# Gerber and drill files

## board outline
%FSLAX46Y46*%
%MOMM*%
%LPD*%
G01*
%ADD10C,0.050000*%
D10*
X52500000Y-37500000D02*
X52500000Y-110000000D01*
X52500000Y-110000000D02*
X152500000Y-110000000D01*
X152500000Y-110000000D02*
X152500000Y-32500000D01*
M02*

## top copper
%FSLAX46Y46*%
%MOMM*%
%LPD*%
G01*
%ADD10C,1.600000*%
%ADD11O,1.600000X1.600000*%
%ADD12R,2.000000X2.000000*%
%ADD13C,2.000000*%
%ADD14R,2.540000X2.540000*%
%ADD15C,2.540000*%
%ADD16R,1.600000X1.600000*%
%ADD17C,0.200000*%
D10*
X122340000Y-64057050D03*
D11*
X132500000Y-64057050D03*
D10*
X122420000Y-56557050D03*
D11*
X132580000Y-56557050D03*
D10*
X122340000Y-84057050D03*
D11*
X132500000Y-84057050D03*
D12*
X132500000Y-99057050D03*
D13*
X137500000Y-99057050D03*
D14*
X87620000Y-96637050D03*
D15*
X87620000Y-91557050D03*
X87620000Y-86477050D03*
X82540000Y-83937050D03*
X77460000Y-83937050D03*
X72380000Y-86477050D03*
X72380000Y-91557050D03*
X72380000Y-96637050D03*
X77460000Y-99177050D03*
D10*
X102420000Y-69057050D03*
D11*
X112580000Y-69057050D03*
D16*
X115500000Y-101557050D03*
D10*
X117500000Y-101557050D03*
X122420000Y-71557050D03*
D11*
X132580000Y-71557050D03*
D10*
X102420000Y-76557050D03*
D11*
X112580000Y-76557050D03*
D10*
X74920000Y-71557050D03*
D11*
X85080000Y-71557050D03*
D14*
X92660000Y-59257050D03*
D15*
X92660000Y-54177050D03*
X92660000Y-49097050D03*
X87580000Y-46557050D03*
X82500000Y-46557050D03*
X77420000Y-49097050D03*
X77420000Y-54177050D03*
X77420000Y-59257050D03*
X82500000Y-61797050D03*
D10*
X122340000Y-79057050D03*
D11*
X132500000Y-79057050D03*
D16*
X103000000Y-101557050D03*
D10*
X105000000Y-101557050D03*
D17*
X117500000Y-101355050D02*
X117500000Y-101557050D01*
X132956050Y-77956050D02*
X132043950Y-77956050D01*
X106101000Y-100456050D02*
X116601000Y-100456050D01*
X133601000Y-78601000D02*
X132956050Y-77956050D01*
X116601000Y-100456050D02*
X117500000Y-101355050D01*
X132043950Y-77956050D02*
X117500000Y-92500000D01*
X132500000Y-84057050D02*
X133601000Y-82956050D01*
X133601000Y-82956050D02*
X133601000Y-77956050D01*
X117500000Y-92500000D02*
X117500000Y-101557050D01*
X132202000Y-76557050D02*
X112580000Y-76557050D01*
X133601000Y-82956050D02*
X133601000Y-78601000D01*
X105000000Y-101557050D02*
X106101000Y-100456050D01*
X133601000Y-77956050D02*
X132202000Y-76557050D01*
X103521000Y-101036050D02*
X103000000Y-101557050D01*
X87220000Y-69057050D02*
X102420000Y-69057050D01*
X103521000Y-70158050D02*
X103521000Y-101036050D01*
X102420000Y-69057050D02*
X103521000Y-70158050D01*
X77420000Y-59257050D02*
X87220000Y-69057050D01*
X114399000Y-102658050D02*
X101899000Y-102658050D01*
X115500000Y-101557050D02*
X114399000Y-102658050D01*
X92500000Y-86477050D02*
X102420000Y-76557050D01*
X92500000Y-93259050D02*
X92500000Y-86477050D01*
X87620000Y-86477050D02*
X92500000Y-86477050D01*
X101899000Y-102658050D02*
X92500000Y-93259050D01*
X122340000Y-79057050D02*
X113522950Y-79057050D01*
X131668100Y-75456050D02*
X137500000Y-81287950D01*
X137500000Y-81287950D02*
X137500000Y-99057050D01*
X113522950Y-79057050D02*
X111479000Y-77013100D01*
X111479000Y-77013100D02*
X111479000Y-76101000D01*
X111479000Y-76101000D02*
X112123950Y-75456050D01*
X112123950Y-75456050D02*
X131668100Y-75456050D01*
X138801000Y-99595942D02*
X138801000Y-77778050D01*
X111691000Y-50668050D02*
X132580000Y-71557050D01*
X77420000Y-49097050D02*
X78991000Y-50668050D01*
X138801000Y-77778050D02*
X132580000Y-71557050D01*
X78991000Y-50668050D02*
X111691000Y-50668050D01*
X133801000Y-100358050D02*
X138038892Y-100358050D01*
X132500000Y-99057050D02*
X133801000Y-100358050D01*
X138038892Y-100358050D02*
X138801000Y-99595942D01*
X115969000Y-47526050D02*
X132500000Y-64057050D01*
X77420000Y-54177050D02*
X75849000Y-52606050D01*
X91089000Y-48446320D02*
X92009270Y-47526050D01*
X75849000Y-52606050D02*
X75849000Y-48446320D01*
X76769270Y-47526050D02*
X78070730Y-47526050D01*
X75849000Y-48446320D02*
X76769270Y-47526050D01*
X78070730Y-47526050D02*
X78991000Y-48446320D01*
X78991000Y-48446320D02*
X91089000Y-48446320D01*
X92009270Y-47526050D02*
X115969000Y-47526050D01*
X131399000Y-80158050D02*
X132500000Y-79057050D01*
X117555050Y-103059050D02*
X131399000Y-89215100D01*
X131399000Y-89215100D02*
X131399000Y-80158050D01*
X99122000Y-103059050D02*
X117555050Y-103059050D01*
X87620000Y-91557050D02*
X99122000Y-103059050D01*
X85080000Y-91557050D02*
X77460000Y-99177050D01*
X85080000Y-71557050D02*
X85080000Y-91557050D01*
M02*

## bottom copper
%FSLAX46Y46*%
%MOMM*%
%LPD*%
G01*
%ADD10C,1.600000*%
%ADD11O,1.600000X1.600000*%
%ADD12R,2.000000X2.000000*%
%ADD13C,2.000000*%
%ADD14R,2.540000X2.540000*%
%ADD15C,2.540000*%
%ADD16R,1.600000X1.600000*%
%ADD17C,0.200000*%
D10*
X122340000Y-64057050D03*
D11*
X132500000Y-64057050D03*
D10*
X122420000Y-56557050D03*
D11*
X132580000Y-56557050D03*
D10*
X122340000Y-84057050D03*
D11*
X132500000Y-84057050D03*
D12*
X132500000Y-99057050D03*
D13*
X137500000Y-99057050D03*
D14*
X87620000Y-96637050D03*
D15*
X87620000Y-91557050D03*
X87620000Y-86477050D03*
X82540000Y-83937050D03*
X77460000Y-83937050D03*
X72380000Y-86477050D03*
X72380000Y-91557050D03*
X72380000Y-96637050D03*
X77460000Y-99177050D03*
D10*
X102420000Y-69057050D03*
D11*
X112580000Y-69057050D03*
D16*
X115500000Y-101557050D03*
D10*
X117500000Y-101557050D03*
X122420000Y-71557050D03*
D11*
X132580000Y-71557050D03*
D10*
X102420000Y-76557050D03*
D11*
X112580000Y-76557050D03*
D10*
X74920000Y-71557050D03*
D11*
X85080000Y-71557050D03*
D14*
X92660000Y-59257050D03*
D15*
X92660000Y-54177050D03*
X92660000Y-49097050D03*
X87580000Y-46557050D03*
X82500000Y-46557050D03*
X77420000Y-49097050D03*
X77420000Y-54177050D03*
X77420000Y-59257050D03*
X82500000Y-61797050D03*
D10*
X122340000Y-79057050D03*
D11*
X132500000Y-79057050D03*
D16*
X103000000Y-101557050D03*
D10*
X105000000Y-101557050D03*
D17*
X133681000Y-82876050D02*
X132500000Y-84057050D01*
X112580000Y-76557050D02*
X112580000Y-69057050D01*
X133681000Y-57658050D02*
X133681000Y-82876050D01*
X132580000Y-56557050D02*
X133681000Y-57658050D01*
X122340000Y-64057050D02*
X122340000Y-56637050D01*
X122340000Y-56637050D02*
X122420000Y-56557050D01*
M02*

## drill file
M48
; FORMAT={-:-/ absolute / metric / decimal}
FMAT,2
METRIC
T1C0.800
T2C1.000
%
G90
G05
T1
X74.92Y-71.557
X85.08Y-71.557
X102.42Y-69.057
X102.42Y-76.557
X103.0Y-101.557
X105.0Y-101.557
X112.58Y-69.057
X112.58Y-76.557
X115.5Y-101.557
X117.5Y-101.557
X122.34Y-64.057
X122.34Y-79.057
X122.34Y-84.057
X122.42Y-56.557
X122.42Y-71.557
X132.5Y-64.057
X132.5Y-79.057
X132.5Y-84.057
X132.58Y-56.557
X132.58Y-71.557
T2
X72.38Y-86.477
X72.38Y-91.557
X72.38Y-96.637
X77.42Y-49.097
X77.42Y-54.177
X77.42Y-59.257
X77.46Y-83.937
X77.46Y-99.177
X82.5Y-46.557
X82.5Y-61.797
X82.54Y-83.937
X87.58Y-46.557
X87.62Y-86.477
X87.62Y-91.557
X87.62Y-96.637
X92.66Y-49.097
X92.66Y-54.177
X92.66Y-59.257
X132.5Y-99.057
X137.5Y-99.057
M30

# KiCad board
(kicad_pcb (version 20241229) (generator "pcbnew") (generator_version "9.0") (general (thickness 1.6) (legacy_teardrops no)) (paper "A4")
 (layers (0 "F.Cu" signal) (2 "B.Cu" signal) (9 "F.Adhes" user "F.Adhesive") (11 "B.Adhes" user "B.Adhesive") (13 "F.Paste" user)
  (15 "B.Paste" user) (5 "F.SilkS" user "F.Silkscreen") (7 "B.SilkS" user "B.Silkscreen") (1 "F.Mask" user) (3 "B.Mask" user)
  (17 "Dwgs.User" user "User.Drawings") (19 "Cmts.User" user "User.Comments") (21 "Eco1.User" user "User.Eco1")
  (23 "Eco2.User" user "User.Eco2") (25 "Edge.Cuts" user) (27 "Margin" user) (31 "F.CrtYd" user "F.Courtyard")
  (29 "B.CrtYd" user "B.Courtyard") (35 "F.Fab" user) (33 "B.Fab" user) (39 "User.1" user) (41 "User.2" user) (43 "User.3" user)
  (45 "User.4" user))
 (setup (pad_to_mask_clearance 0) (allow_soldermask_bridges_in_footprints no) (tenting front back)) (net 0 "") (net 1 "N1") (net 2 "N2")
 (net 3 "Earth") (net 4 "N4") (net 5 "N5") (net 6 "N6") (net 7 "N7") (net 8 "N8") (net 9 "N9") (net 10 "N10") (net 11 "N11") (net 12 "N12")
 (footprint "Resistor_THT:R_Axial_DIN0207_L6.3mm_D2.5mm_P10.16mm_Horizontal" (layer "F.Cu") (at 122.34 64.05705)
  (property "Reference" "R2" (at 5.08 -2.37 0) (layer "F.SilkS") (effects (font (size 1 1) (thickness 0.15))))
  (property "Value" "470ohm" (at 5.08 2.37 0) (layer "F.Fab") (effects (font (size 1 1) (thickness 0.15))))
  (pad "1" thru_hole circle (at 0 0) (size 1.6 1.6) (drill 0.8) (layers "*.Cu" "*.Mask") (remove_unused_layers no) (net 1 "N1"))
  (pad "2" thru_hole oval (at 10.16 0) (size 1.6 1.6) (drill 0.8) (layers "*.Cu" "*.Mask") (remove_unused_layers no) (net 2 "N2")))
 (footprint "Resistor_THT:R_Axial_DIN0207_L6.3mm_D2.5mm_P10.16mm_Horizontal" (layer "F.Cu") (at 122.42 56.55705)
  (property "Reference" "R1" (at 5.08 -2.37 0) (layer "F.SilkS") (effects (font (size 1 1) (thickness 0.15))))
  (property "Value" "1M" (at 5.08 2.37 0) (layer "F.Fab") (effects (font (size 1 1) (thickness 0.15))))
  (pad "1" thru_hole circle (at 0 0) (size 1.6 1.6) (drill 0.8) (layers "*.Cu" "*.Mask") (remove_unused_layers no) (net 1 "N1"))
  (pad "2" thru_hole oval (at 10.16 0) (size 1.6 1.6) (drill 0.8) (layers "*.Cu" "*.Mask") (remove_unused_layers no) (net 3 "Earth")))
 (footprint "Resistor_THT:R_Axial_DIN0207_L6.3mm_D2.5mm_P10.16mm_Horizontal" (layer "F.Cu") (at 122.34 84.05705)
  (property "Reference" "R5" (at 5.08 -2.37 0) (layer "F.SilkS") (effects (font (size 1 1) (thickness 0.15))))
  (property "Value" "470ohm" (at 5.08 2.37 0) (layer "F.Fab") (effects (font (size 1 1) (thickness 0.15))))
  (pad "1" thru_hole circle (at 0 0) (size 1.6 1.6) (drill 0.8) (layers "*.Cu" "*.Mask") (remove_unused_layers no) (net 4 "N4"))
  (pad "2" thru_hole oval (at 10.16 0) (size 1.6 1.6) (drill 0.8) (layers "*.Cu" "*.Mask") (remove_unused_layers no) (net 3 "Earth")))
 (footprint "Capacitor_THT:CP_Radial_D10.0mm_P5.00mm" (layer "F.Cu") (at 132.5 99.05705)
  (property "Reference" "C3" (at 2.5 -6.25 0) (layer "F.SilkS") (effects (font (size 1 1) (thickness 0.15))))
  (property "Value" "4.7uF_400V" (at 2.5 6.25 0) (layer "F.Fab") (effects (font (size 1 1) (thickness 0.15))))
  (pad "1" thru_hole rect (at 0 0) (size 2 2) (drill 1) (layers "*.Cu" "*.Mask") (remove_unused_layers no) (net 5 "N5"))
  (pad "2" thru_hole circle (at 5 0) (size 2 2) (drill 1) (layers "*.Cu" "*.Mask") (remove_unused_layers no) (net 4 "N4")))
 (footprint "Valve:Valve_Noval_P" (layer "F.Cu") (at 87.62 96.63705)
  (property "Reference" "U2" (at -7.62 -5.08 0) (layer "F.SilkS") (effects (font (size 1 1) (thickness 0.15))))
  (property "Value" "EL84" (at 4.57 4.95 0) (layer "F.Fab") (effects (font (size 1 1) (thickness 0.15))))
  (pad "1" thru_hole rect (at 0 0) (size 2.54 2.54) (drill 1) (layers "*.Cu" "*.Mask") (remove_unused_layers no))
  (pad "2" thru_hole circle (at 0 -5.08) (size 2.54 2.54) (drill 1) (layers "*.Cu" "*.Mask") (remove_unused_layers no) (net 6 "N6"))
  (pad "3" thru_hole circle (at 0 -10.16) (size 2.54 2.54) (drill 1) (layers "*.Cu" "*.Mask") (remove_unused_layers no) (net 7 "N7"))
  (pad "4" thru_hole circle (at -5.08 -12.7) (size 2.54 2.54) (drill 1) (layers "*.Cu" "*.Mask") (remove_unused_layers no))
  (pad "5" thru_hole circle (at -10.16 -12.7) (size 2.54 2.54) (drill 1) (layers "*.Cu" "*.Mask") (remove_unused_layers no))
  (pad "6" thru_hole circle (at -15.24 -10.16) (size 2.54 2.54) (drill 1) (layers "*.Cu" "*.Mask") (remove_unused_layers no))
  (pad "7" thru_hole circle (at -15.24 -5.08) (size 2.54 2.54) (drill 1) (layers "*.Cu" "*.Mask") (remove_unused_layers no) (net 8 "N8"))
  (pad "8" thru_hole circle (at -15.24 0) (size 2.54 2.54) (drill 1) (layers "*.Cu" "*.Mask") (remove_unused_layers no))
  (pad "9" thru_hole circle (at -10.16 2.54) (size 2.54 2.54) (drill 1) (layers "*.Cu" "*.Mask") (remove_unused_layers no) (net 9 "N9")))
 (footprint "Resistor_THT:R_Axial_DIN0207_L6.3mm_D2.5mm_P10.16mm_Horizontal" (layer "F.Cu") (at 102.42 69.05705)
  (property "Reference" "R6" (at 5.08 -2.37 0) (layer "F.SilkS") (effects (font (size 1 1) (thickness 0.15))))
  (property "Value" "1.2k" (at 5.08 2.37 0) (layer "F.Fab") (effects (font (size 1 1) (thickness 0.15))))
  (pad "1" thru_hole circle (at 0 0) (size 1.6 1.6) (drill 0.8) (layers "*.Cu" "*.Mask") (remove_unused_layers no) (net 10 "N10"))
  (pad "2" thru_hole oval (at 10.16 0) (size 1.6 1.6) (drill 0.8) (layers "*.Cu" "*.Mask") (remove_unused_layers no) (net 3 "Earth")))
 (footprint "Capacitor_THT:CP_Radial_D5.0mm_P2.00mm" (layer "F.Cu") (at 115.5 101.55705)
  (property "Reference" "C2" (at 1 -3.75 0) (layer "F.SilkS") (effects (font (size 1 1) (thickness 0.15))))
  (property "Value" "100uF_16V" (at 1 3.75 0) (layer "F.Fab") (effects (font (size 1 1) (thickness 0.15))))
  (pad "1" thru_hole rect (at 0 0) (size 1.6 1.6) (drill 0.8) (layers "*.Cu" "*.Mask") (remove_unused_layers no) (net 7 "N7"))
  (pad "2" thru_hole circle (at 2 0) (size 1.6 1.6) (drill 0.8) (layers "*.Cu" "*.Mask") (remove_unused_layers no) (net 3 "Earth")))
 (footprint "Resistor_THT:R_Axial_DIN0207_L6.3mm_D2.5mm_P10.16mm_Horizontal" (layer "F.Cu") (at 122.42 71.55705)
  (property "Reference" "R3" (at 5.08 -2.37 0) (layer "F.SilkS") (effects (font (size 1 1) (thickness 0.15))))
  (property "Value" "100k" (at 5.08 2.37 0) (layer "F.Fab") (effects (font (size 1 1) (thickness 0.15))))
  (pad "1" thru_hole circle (at 0 0) (size 1.6 1.6) (drill 0.8) (layers "*.Cu" "*.Mask") (remove_unused_layers no) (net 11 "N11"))
  (pad "2" thru_hole oval (at 10.16 0) (size 1.6 1.6) (drill 0.8) (layers "*.Cu" "*.Mask") (remove_unused_layers no) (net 5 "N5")))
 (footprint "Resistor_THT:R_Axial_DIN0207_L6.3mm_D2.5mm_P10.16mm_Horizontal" (layer "F.Cu") (at 102.42 76.55705)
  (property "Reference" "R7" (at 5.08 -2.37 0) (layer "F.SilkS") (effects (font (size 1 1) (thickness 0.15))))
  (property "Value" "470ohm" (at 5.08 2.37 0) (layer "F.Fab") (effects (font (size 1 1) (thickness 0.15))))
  (pad "1" thru_hole circle (at 0 0) (size 1.6 1.6) (drill 0.8) (layers "*.Cu" "*.Mask") (remove_unused_layers no) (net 7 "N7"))
  (pad "2" thru_hole oval (at 10.16 0) (size 1.6 1.6) (drill 0.8) (layers "*.Cu" "*.Mask") (remove_unused_layers no) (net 3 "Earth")))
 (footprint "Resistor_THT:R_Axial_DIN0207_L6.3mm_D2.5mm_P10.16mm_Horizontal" (layer "F.Cu") (at 74.92 71.55705)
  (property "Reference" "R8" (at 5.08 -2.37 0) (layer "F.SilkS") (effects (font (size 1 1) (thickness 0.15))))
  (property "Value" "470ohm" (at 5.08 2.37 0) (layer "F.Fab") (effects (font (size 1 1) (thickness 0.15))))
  (pad "1" thru_hole circle (at 0 0) (size 1.6 1.6) (drill 0.8) (layers "*.Cu" "*.Mask") (remove_unused_layers no) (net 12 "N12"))
  (pad "2" thru_hole oval (at 10.16 0) (size 1.6 1.6) (drill 0.8) (layers "*.Cu" "*.Mask") (remove_unused_layers no) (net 9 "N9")))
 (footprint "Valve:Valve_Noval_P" (layer "F.Cu") (at 92.66 59.25705)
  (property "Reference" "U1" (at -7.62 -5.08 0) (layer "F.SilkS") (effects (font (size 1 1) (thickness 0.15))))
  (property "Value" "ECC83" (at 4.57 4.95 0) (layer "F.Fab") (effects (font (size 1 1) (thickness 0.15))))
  (pad "1" thru_hole rect (at 0 0) (size 2.54 2.54) (drill 1) (layers "*.Cu" "*.Mask") (remove_unused_layers no))
  (pad "2" thru_hole circle (at 0 -5.08) (size 2.54 2.54) (drill 1) (layers "*.Cu" "*.Mask") (remove_unused_layers no))
  (pad "3" thru_hole circle (at 0 -10.16) (size 2.54 2.54) (drill 1) (layers "*.Cu" "*.Mask") (remove_unused_layers no))
  (pad "4" thru_hole circle (at -5.08 -12.7) (size 2.54 2.54) (drill 1) (layers "*.Cu" "*.Mask") (remove_unused_layers no))
  (pad "5" thru_hole circle (at -10.16 -12.7) (size 2.54 2.54) (drill 1) (layers "*.Cu" "*.Mask") (remove_unused_layers no))
  (pad "6" thru_hole circle (at -15.24 -10.16) (size 2.54 2.54) (drill 1) (layers "*.Cu" "*.Mask") (remove_unused_layers no) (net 5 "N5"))
  (pad "7" thru_hole circle (at -15.24 -5.08) (size 2.54 2.54) (drill 1) (layers "*.Cu" "*.Mask") (remove_unused_layers no) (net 2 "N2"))
  (pad "8" thru_hole circle (at -15.24 0) (size 2.54 2.54) (drill 1) (layers "*.Cu" "*.Mask") (remove_unused_layers no) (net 10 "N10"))
  (pad "9" thru_hole circle (at -10.16 2.54) (size 2.54 2.54) (drill 1) (layers "*.Cu" "*.Mask") (remove_unused_layers no)))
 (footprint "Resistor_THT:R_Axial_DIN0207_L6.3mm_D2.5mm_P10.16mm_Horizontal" (layer "F.Cu") (at 122.34 79.05705)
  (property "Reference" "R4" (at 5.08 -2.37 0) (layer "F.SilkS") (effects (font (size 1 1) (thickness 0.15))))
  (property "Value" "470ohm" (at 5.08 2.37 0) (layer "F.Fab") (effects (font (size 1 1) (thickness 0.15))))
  (pad "1" thru_hole circle (at 0 0) (size 1.6 1.6) (drill 0.8) (layers "*.Cu" "*.Mask") (remove_unused_layers no) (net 4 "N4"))
  (pad "2" thru_hole oval (at 10.16 0) (size 1.6 1.6) (drill 0.8) (layers "*.Cu" "*.Mask") (remove_unused_layers no) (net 6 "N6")))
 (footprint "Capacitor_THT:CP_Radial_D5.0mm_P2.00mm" (layer "F.Cu") (at 103 101.55705)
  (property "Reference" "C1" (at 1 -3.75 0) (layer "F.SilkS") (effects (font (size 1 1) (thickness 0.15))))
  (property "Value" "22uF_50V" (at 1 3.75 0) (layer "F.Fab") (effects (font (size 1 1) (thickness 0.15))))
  (pad "1" thru_hole rect (at 0 0) (size 1.6 1.6) (drill 0.8) (layers "*.Cu" "*.Mask") (remove_unused_layers no) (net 10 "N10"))
  (pad "2" thru_hole circle (at 2 0) (size 1.6 1.6) (drill 0.8) (layers "*.Cu" "*.Mask") (remove_unused_layers no) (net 3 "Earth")))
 (gr_line (start 52.5 37.5) (end 52.5 110) (stroke (width 0.05) (type default)) (layer "Edge.Cuts"))
 (gr_line (start 52.5 110) (end 152.5 110) (stroke (width 0.05) (type default)) (layer "Edge.Cuts"))
 (gr_line (start 152.5 110) (end 152.5 32.5) (stroke (width 0.05) (type default)) (layer "Edge.Cuts"))
 (segment (start 117.5 101.35505) (end 117.5 101.55705) (width 0.2) (layer "F.Cu") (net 3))
 (segment (start 132.95605 77.95605) (end 132.04395 77.95605) (width 0.2) (layer "F.Cu") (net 3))
 (segment (start 106.101 100.45605) (end 116.601 100.45605) (width 0.2) (layer "F.Cu") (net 3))
 (segment (start 133.601 78.601) (end 132.95605 77.95605) (width 0.2) (layer "F.Cu") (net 3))
 (segment (start 116.601 100.45605) (end 117.5 101.35505) (width 0.2) (layer "F.Cu") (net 3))
 (segment (start 132.04395 77.95605) (end 117.5 92.5) (width 0.2) (layer "F.Cu") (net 3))
 (segment (start 132.5 84.05705) (end 133.601 82.95605) (width 0.2) (layer "F.Cu") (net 3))
 (segment (start 133.601 82.95605) (end 133.601 77.95605) (width 0.2) (layer "F.Cu") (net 3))
 (segment (start 117.5 92.5) (end 117.5 101.55705) (width 0.2) (layer "F.Cu") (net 3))
 (segment (start 132.202 76.55705) (end 112.58 76.55705) (width 0.2) (layer "F.Cu") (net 3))
 (segment (start 133.601 82.95605) (end 133.601 78.601) (width 0.2) (layer "F.Cu") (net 3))
 (segment (start 105 101.55705) (end 106.101 100.45605) (width 0.2) (layer "F.Cu") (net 3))
 (segment (start 133.601 77.95605) (end 132.202 76.55705) (width 0.2) (layer "F.Cu") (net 3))
 (segment (start 133.681 82.87605) (end 132.5 84.05705) (width 0.2) (layer "B.Cu") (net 3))
 (segment (start 112.58 76.55705) (end 112.58 69.05705) (width 0.2) (layer "B.Cu") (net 3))
 (segment (start 133.681 57.65805) (end 133.681 82.87605) (width 0.2) (layer "B.Cu") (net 3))
 (segment (start 132.58 56.55705) (end 133.681 57.65805) (width 0.2) (layer "B.Cu") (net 3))
 (segment (start 103.521 101.03605) (end 103 101.55705) (width 0.2) (layer "F.Cu") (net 10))
 (segment (start 87.22 69.05705) (end 102.42 69.05705) (width 0.2) (layer "F.Cu") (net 10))
 (segment (start 103.521 70.15805) (end 103.521 101.03605) (width 0.2) (layer "F.Cu") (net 10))
 (segment (start 102.42 69.05705) (end 103.521 70.15805) (width 0.2) (layer "F.Cu") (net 10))
 (segment (start 77.42 59.25705) (end 87.22 69.05705) (width 0.2) (layer "F.Cu") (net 10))
 (segment (start 114.399 102.65805) (end 101.899 102.65805) (width 0.2) (layer "F.Cu") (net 7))
 (segment (start 115.5 101.55705) (end 114.399 102.65805) (width 0.2) (layer "F.Cu") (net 7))
 (segment (start 92.5 86.47705) (end 102.42 76.55705) (width 0.2) (layer "F.Cu") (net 7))
 (segment (start 92.5 93.25905) (end 92.5 86.47705) (width 0.2) (layer "F.Cu") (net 7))
 (segment (start 87.62 86.47705) (end 92.5 86.47705) (width 0.2) (layer "F.Cu") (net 7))
 (segment (start 101.899 102.65805) (end 92.5 93.25905) (width 0.2) (layer "F.Cu") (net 7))
 (segment (start 122.34 79.05705) (end 113.52295 79.05705) (width 0.2) (layer "F.Cu") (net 4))
 (segment (start 131.6681 75.45605) (end 137.5 81.28795) (width 0.2) (layer "F.Cu") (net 4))
 (segment (start 137.5 81.28795) (end 137.5 99.05705) (width 0.2) (layer "F.Cu") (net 4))
 (segment (start 113.52295 79.05705) (end 111.479 77.0131) (width 0.2) (layer "F.Cu") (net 4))
 (segment (start 111.479 77.0131) (end 111.479 76.101) (width 0.2) (layer "F.Cu") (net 4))
 (segment (start 111.479 76.101) (end 112.12395 75.45605) (width 0.2) (layer "F.Cu") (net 4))
 (segment (start 112.12395 75.45605) (end 131.6681 75.45605) (width 0.2) (layer "F.Cu") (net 4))
 (segment (start 138.801 99.595942) (end 138.801 77.77805) (width 0.2) (layer "F.Cu") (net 5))
 (segment (start 111.691 50.66805) (end 132.58 71.55705) (width 0.2) (layer "F.Cu") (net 5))
 (segment (start 77.42 49.09705) (end 78.991 50.66805) (width 0.2) (layer "F.Cu") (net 5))
 (segment (start 138.801 77.77805) (end 132.58 71.55705) (width 0.2) (layer "F.Cu") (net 5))
 (segment (start 78.991 50.66805) (end 111.691 50.66805) (width 0.2) (layer "F.Cu") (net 5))
 (segment (start 133.801 100.35805) (end 138.038892 100.35805) (width 0.2) (layer "F.Cu") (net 5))
 (segment (start 132.5 99.05705) (end 133.801 100.35805) (width 0.2) (layer "F.Cu") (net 5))
 (segment (start 138.038892 100.35805) (end 138.801 99.595942) (width 0.2) (layer "F.Cu") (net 5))
 (segment (start 122.34 64.05705) (end 122.34 56.63705) (width 0.2) (layer "B.Cu") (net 1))
 (segment (start 122.34 56.63705) (end 122.42 56.55705) (width 0.2) (layer "B.Cu") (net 1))
 (segment (start 115.969 47.52605) (end 132.5 64.05705) (width 0.2) (layer "F.Cu") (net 2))
 (segment (start 77.42 54.17705) (end 75.849 52.60605) (width 0.2) (layer "F.Cu") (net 2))
 (segment (start 91.089 48.44632) (end 92.00927 47.52605) (width 0.2) (layer "F.Cu") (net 2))
 (segment (start 75.849 52.60605) (end 75.849 48.44632) (width 0.2) (layer "F.Cu") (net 2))
 (segment (start 76.76927 47.52605) (end 78.07073 47.52605) (width 0.2) (layer "F.Cu") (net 2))
 (segment (start 75.849 48.44632) (end 76.76927 47.52605) (width 0.2) (layer "F.Cu") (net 2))
 (segment (start 78.07073 47.52605) (end 78.991 48.44632) (width 0.2) (layer "F.Cu") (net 2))
 (segment (start 78.991 48.44632) (end 91.089 48.44632) (width 0.2) (layer "F.Cu") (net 2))
 (segment (start 92.00927 47.52605) (end 115.969 47.52605) (width 0.2) (layer "F.Cu") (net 2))
 (segment (start 131.399 80.15805) (end 132.5 79.05705) (width 0.2) (layer "F.Cu") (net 6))
 (segment (start 117.55505 103.05905) (end 131.399 89.2151) (width 0.2) (layer "F.Cu") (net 6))
 (segment (start 131.399 89.2151) (end 131.399 80.15805) (width 0.2) (layer "F.Cu") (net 6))
 (segment (start 99.122 103.05905) (end 117.55505 103.05905) (width 0.2) (layer "F.Cu") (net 6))
 (segment (start 87.62 91.55705) (end 99.122 103.05905) (width 0.2) (layer "F.Cu") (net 6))
 (segment (start 85.08 91.55705) (end 77.46 99.17705) (width 0.2) (layer "F.Cu") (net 9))
 (segment (start 85.08 71.55705) (end 85.08 91.55705) (width 0.2) (layer "F.Cu") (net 9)))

